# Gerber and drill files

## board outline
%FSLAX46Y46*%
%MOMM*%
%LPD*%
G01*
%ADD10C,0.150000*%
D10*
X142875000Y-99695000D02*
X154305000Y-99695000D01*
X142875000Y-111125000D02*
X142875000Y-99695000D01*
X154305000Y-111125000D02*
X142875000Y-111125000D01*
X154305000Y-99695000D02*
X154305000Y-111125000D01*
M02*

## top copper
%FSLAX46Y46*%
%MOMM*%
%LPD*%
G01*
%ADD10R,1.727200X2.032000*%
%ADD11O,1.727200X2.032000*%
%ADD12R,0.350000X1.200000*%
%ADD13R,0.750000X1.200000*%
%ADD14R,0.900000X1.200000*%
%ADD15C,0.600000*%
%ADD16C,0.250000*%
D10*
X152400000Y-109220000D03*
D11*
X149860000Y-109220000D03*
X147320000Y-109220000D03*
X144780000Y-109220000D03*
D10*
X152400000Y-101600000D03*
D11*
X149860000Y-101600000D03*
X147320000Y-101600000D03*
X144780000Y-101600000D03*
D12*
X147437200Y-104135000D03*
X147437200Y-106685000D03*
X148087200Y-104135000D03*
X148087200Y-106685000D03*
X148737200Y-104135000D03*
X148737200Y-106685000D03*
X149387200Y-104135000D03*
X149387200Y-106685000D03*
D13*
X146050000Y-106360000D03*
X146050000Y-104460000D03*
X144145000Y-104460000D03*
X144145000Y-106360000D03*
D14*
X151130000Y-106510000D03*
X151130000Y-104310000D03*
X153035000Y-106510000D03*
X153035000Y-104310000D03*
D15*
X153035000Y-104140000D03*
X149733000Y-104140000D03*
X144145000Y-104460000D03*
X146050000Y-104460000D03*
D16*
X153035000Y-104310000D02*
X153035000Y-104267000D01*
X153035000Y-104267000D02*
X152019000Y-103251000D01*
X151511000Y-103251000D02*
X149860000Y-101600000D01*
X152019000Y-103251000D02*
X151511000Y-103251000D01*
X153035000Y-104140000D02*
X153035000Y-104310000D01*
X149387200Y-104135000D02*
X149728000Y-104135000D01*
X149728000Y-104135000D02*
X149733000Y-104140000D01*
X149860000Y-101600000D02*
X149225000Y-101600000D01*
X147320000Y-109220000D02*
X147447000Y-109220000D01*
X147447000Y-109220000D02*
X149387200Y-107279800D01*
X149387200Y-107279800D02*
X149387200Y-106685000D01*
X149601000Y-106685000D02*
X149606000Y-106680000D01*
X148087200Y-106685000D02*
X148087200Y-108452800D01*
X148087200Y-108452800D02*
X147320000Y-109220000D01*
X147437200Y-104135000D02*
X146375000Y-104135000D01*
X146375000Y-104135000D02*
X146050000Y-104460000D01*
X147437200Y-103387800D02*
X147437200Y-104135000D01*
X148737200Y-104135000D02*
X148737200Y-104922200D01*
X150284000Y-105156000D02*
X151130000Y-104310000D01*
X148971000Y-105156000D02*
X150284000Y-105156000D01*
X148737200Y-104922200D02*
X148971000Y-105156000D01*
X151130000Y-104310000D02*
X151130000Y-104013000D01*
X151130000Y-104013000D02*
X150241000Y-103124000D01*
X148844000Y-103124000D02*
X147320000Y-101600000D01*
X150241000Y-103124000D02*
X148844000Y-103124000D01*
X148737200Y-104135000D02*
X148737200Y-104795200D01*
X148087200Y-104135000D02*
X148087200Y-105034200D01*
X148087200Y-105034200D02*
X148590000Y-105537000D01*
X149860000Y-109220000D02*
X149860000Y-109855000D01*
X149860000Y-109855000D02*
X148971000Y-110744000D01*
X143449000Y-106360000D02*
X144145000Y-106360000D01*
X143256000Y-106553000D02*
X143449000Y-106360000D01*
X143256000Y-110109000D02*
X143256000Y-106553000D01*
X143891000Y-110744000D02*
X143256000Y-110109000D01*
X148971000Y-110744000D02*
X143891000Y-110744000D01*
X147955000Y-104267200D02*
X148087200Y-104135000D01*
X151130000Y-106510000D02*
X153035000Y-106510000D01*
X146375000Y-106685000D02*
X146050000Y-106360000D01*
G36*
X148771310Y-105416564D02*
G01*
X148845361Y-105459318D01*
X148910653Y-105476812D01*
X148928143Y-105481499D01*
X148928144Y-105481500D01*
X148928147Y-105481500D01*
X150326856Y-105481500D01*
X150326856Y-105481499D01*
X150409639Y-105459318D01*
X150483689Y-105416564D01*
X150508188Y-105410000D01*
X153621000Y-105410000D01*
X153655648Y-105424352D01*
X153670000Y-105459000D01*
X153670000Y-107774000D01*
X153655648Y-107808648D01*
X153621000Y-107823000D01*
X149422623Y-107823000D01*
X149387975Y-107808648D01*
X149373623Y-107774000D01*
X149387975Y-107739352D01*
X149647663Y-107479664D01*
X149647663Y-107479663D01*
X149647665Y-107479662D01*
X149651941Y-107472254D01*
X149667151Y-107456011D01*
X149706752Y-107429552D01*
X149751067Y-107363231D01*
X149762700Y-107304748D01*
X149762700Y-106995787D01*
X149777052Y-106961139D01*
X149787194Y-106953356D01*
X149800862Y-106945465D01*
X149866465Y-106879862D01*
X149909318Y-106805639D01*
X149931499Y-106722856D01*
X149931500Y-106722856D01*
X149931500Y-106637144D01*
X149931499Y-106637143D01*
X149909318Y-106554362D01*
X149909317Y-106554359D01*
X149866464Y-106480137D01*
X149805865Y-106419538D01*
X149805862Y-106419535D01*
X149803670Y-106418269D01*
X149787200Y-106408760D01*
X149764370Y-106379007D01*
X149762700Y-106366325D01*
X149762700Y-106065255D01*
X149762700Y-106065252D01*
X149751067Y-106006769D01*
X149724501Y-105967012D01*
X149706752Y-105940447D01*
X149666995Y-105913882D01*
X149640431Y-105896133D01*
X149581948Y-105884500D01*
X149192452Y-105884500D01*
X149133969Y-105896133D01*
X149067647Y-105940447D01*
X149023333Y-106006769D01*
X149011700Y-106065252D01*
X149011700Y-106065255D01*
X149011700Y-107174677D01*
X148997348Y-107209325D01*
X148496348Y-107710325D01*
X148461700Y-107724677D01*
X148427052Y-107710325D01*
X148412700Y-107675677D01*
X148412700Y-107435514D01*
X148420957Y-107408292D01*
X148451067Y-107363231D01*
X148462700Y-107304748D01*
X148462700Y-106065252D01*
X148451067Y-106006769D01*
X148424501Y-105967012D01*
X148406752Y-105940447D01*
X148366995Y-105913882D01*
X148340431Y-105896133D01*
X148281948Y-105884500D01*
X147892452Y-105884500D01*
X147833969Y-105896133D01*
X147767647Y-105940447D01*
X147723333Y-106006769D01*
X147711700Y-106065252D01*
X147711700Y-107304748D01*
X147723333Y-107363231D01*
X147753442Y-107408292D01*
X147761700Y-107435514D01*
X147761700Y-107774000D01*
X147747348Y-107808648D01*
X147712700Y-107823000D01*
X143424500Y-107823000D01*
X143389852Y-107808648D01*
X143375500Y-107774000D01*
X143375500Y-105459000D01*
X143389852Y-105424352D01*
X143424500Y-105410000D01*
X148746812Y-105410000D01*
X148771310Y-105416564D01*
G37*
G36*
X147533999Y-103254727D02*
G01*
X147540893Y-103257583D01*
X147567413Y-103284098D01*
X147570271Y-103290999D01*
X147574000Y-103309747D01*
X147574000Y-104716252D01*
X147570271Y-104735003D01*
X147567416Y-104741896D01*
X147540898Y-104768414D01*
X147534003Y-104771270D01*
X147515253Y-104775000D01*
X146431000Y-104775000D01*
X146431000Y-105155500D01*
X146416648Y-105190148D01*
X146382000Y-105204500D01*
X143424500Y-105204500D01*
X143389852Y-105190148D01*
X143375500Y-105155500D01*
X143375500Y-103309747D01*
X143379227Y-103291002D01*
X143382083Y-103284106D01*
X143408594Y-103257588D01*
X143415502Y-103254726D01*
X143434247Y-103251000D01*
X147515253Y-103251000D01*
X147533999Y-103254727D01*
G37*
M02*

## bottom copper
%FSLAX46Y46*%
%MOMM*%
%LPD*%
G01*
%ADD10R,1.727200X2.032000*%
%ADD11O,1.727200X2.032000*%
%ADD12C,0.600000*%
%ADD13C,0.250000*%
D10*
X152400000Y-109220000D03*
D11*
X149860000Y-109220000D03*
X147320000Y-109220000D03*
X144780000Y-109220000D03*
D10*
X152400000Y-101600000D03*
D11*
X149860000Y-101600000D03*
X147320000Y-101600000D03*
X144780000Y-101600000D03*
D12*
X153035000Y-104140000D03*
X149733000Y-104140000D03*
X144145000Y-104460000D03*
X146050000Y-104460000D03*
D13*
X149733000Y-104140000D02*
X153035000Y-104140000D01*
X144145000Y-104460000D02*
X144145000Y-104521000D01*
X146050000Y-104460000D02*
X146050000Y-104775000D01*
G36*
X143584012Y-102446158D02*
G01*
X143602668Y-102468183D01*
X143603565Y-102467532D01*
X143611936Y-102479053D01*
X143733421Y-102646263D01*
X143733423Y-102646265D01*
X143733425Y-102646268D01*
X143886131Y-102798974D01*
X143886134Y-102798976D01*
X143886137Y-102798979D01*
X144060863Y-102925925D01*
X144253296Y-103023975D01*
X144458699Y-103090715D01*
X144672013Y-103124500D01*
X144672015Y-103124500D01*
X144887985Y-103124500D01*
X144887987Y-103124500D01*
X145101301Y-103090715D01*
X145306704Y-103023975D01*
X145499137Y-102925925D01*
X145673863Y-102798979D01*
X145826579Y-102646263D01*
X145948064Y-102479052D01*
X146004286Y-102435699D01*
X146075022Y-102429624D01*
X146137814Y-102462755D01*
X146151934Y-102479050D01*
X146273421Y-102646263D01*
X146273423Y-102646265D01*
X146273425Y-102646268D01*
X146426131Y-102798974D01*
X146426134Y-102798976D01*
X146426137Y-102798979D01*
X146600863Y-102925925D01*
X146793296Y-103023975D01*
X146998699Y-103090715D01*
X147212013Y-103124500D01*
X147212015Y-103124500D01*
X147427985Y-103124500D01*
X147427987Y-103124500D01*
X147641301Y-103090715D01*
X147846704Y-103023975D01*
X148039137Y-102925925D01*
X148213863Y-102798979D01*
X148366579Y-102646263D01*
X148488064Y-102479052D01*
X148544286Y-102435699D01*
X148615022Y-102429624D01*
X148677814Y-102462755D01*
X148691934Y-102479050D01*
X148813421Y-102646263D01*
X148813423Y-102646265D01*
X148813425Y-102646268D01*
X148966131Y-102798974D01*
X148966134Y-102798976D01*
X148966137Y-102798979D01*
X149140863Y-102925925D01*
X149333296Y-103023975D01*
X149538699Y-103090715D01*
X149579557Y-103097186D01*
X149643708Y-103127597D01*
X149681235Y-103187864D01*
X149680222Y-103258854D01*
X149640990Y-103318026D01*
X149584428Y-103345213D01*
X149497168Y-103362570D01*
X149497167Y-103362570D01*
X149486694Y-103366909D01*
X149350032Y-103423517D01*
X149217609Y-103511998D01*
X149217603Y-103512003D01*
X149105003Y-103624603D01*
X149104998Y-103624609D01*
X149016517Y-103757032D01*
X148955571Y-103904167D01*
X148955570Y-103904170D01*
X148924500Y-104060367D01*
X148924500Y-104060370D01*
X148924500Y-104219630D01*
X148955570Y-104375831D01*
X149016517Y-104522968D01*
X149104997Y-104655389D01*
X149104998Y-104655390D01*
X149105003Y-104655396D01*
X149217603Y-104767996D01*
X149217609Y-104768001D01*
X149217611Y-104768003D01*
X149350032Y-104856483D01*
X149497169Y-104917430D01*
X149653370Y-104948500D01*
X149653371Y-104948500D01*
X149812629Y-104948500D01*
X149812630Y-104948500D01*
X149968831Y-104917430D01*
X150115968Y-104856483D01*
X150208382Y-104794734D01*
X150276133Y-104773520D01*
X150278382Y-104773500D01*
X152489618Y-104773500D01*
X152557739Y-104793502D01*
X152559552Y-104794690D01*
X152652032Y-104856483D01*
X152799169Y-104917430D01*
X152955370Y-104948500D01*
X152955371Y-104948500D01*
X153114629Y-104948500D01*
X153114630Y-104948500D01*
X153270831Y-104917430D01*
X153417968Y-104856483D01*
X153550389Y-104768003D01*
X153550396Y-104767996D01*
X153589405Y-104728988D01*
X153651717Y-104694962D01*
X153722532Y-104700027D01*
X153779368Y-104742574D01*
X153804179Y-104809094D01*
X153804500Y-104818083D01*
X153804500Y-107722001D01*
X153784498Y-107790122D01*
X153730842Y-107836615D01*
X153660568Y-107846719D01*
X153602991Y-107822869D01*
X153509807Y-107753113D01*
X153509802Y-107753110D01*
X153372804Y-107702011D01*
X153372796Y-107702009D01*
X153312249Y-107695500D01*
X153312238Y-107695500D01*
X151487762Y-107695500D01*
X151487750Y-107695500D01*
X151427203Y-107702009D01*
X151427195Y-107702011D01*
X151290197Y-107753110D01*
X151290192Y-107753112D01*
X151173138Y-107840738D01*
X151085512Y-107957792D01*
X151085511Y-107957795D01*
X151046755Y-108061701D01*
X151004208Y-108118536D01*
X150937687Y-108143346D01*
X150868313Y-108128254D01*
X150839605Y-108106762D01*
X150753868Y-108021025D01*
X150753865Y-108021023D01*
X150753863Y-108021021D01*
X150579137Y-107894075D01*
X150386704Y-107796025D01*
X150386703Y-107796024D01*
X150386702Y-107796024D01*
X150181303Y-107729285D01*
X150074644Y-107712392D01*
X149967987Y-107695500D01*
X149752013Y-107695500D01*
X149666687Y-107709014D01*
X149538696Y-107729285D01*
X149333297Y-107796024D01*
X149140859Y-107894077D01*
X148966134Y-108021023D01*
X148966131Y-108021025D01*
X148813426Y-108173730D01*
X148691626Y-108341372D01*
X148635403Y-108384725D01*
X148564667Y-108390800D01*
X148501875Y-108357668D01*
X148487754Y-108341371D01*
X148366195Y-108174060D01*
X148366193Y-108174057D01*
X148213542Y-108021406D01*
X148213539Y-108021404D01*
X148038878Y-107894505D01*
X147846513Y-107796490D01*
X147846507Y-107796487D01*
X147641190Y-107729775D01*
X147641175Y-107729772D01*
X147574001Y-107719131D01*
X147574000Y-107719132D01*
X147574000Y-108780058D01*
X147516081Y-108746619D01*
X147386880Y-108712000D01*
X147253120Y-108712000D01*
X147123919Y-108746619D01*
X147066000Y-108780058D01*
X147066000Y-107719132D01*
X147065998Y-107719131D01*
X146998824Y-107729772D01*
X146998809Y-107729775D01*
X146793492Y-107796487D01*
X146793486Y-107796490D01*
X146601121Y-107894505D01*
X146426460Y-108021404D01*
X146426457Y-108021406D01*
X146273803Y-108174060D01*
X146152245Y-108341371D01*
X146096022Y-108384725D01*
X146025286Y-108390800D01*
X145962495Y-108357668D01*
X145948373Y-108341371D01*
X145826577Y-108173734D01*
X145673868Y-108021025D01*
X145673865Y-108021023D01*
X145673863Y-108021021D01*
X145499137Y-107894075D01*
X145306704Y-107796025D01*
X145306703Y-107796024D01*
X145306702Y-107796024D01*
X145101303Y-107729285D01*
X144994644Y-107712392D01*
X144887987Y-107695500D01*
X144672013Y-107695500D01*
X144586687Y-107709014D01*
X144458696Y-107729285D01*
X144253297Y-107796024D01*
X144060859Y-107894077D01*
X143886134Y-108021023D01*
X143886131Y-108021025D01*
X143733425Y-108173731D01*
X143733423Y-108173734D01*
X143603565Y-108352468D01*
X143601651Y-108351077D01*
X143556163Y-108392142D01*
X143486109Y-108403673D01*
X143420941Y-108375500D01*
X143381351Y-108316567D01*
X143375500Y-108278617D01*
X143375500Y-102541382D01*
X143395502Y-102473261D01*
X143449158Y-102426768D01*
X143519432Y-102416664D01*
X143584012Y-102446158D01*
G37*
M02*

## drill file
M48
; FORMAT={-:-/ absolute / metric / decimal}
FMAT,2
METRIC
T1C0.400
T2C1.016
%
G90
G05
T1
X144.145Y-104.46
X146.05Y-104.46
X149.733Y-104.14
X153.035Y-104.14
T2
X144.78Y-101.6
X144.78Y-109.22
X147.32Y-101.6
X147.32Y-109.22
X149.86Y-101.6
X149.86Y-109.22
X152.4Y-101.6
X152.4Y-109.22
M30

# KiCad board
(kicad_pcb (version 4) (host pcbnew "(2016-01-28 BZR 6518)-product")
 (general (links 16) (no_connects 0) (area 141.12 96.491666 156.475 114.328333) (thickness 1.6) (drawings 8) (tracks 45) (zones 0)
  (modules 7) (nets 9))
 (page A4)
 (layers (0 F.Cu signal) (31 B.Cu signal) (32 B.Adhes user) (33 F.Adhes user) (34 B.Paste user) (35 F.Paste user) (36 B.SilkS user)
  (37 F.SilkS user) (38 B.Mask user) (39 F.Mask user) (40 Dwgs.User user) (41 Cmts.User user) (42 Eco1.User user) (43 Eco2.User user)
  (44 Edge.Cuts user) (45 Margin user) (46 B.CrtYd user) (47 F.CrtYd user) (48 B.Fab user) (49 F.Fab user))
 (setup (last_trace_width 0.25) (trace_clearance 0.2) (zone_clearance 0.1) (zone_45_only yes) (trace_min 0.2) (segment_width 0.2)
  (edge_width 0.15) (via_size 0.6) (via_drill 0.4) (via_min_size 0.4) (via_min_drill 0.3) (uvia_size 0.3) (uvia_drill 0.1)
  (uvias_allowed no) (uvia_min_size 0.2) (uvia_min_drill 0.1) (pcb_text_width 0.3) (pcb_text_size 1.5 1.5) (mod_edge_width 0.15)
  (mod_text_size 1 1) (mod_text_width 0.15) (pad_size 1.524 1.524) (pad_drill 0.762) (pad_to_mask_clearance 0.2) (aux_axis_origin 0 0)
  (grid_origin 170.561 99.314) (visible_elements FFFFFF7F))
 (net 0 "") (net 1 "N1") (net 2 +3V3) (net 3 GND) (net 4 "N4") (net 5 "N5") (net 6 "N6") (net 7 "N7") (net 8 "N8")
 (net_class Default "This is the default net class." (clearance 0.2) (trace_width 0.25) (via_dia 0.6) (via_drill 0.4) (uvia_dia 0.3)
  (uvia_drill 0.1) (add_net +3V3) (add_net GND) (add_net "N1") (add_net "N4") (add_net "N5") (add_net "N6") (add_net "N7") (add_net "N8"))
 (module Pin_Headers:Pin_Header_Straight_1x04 (layer F.Cu) (at 152.4 109.22 270)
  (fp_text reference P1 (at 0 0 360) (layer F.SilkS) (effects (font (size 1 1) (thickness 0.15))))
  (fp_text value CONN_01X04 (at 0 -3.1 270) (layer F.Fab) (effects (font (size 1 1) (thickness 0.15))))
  (pad 1 thru_hole rect (at 0 0 270) (size 2.032 1.7272) (drill 1.016) (layers *.Cu *.Mask F.SilkS) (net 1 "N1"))
  (pad 2 thru_hole oval (at 0 2.54 270) (size 2.032 1.7272) (drill 1.016) (layers *.Cu *.Mask F.SilkS) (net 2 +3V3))
  (pad 3 thru_hole oval (at 0 5.08 270) (size 2.032 1.7272) (drill 1.016) (layers *.Cu *.Mask F.SilkS) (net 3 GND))
  (pad 4 thru_hole oval (at 0 7.62 270) (size 2.032 1.7272) (drill 1.016) (layers *.Cu *.Mask F.SilkS) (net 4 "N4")))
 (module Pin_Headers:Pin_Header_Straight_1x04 (layer F.Cu) (at 152.4 101.6 270)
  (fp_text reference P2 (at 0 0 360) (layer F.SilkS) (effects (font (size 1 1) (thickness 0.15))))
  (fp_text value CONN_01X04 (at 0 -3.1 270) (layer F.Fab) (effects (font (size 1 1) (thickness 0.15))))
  (pad 1 thru_hole rect (at 0 0 270) (size 2.032 1.7272) (drill 1.016) (layers *.Cu *.Mask F.SilkS) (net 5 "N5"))
  (pad 2 thru_hole oval (at 0 2.54 270) (size 2.032 1.7272) (drill 1.016) (layers *.Cu *.Mask F.SilkS) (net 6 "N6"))
  (pad 3 thru_hole oval (at 0 5.08 270) (size 2.032 1.7272) (drill 1.016) (layers *.Cu *.Mask F.SilkS) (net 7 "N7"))
  (pad 4 thru_hole oval (at 0 7.62 270) (size 2.032 1.7272) (drill 1.016) (layers *.Cu *.Mask F.SilkS) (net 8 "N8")))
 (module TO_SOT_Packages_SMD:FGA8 (layer F.Cu) (at 148.4122 105.41) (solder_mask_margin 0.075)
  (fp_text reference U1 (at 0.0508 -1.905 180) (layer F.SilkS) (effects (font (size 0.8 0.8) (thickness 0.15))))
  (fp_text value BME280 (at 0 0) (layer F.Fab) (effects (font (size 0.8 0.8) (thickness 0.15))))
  (pad 1 smd rect (at -0.975 -1.275) (size 0.35 1.2) (layers F.Cu F.Paste F.Mask) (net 3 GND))
  (pad 8 smd rect (at -0.975 1.275) (size 0.35 1.2) (layers F.Cu F.Paste F.Mask) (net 2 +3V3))
  (pad 2 smd rect (at -0.325 -1.275) (size 0.35 1.2) (layers F.Cu F.Paste F.Mask) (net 2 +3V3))
  (pad 7 smd rect (at -0.325 1.275) (size 0.35 1.2) (layers F.Cu F.Paste F.Mask) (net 3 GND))
  (pad 3 smd rect (at 0.325 -1.275) (size 0.35 1.2) (layers F.Cu F.Paste F.Mask) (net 7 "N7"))
  (pad 6 smd rect (at 0.325 1.275) (size 0.35 1.2) (layers F.Cu F.Paste F.Mask) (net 2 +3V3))
  (pad 4 smd rect (at 0.975 -1.275) (size 0.35 1.2) (layers F.Cu F.Paste F.Mask) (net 6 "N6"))
  (pad 5 smd rect (at 0.975 1.275) (size 0.35 1.2) (layers F.Cu F.Paste F.Mask) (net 3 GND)))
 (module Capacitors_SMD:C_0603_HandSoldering (layer F.Cu) (at 146.05 105.41 90)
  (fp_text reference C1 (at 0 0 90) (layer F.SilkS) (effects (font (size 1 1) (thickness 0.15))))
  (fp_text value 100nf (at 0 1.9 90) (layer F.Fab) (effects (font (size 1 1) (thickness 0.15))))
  (pad 1 smd rect (at -0.95 0 90) (size 1.2 0.75) (layers F.Cu F.Paste F.Mask) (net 2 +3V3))
  (pad 2 smd rect (at 0.95 0 90) (size 1.2 0.75) (layers F.Cu F.Paste F.Mask) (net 3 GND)))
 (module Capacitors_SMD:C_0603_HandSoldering (layer F.Cu) (at 144.145 105.41 270)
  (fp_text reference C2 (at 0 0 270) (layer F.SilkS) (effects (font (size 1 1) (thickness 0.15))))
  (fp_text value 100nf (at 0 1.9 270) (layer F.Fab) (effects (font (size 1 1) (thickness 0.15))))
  (pad 1 smd rect (at -0.95 0 270) (size 1.2 0.75) (layers F.Cu F.Paste F.Mask) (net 3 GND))
  (pad 2 smd rect (at 0.95 0 270) (size 1.2 0.75) (layers F.Cu F.Paste F.Mask) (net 2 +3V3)))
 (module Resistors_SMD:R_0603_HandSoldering (layer F.Cu) (at 151.13 105.41 90)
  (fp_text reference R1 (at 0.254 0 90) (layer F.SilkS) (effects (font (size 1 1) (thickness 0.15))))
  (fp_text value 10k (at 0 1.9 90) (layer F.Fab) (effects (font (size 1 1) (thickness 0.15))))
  (pad 1 smd rect (at -1.1 0 90) (size 1.2 0.9) (layers F.Cu F.Paste F.Mask) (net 2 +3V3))
  (pad 2 smd rect (at 1.1 0 90) (size 1.2 0.9) (layers F.Cu F.Paste F.Mask) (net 7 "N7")))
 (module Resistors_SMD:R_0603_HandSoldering (layer F.Cu) (at 153.035 105.41 90)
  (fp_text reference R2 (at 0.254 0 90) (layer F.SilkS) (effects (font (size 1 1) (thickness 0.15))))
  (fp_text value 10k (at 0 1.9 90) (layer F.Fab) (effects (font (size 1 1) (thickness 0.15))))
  (pad 1 smd rect (at -1.1 0 90) (size 1.2 0.9) (layers F.Cu F.Paste F.Mask) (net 2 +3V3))
  (pad 2 smd rect (at 1.1 0 90) (size 1.2 0.9) (layers F.Cu F.Paste F.Mask) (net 6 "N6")))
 (gr_line (start 142.875 99.695) (end 154.305 99.695) (angle 90) (layer Edge.Cuts) (width 0.15))
 (gr_line (start 142.875 111.125) (end 142.875 99.695) (angle 90) (layer Edge.Cuts) (width 0.15))
 (gr_line (start 154.305 111.125) (end 142.875 111.125) (angle 90) (layer Edge.Cuts) (width 0.15))
 (gr_line (start 154.305 99.695) (end 154.305 111.125) (angle 90) (layer Edge.Cuts) (width 0.15))
 (segment (start 153.035 104.31) (end 153.035 104.267) (width 0.25) (layer F.Cu) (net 6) (status C00000))
 (segment (start 153.035 104.267) (end 152.019 103.251) (width 0.25) (layer F.Cu) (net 6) (status 400000))
 (segment (start 151.511 103.251) (end 149.86 101.6) (width 0.25) (layer F.Cu) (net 6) (status 800000))
 (segment (start 152.019 103.251) (end 151.511 103.251) (width 0.25) (layer F.Cu) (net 6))
 (via (at 153.035 104.14) (size 0.6) (drill 0.4) (layers F.Cu B.Cu) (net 6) (status 800000))
 (segment (start 153.035 104.14) (end 153.035 104.31) (width 0.25) (layer F.Cu) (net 6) (status C00000))
 (segment (start 149.3872 104.135) (end 149.728 104.135) (width 0.25) (layer F.Cu) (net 6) (status 400000))
 (segment (start 149.733 104.14) (end 153.035 104.14) (width 0.25) (layer B.Cu) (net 6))
 (via (at 149.733 104.14) (size 0.6) (drill 0.4) (layers F.Cu B.Cu) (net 6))
 (segment (start 149.728 104.135) (end 149.733 104.14) (width 0.25) (layer F.Cu) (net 6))
 (segment (start 149.86 101.6) (end 149.225 101.6) (width 0.25) (layer F.Cu) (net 6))
 (via (at 144.145 104.46) (size 0.6) (drill 0.4) (layers F.Cu B.Cu) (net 3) (status C00000))
 (segment (start 144.145 104.46) (end 144.145 104.521) (width 0.25) (layer B.Cu) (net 3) (status 400000))
 (segment (start 147.32 109.22) (end 147.447 109.22) (width 0.25) (layer F.Cu) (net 3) (status C00000))
 (segment (start 147.447 109.22) (end 149.3872 107.2798) (width 0.25) (layer F.Cu) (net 3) (status C00000))
 (segment (start 149.3872 107.2798) (end 149.3872 106.685) (width 0.25) (layer F.Cu) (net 3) (status C00000))
 (segment (start 149.601 106.685) (end 149.606 106.68) (width 0.25) (layer F.Cu) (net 3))
 (segment (start 148.0872 106.685) (end 148.0872 108.4528) (width 0.25) (layer F.Cu) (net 3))
 (segment (start 148.0872 108.4528) (end 147.32 109.22) (width 0.25) (layer F.Cu) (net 3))
 (segment (start 147.4372 104.135) (end 146.375 104.135) (width 0.25) (layer F.Cu) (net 3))
 (segment (start 146.375 104.135) (end 146.05 104.46) (width 0.25) (layer F.Cu) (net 3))
 (via (at 146.05 104.46) (size 0.6) (drill 0.4) (layers F.Cu B.Cu) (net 3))
 (segment (start 146.05 104.46) (end 146.05 104.775) (width 0.25) (layer B.Cu) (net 3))
 (segment (start 147.4372 103.3878) (end 147.4372 104.135) (width 0.25) (layer F.Cu) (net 3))
 (segment (start 148.7372 104.135) (end 148.7372 104.9222) (width 0.25) (layer F.Cu) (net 7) (status 400000))
 (segment (start 150.284 105.156) (end 151.13 104.31) (width 0.25) (layer F.Cu) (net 7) (status 800000))
 (segment (start 148.971 105.156) (end 150.284 105.156) (width 0.25) (layer F.Cu) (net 7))
 (segment (start 148.7372 104.9222) (end 148.971 105.156) (width 0.25) (layer F.Cu) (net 7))
 (segment (start 151.13 104.31) (end 151.13 104.013) (width 0.25) (layer F.Cu) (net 7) (status C00000))
 (segment (start 151.13 104.013) (end 150.241 103.124) (width 0.25) (layer F.Cu) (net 7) (status 400000))
 (segment (start 148.844 103.124) (end 147.32 101.6) (width 0.25) (layer F.Cu) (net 7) (status 800000))
 (segment (start 150.241 103.124) (end 148.844 103.124) (width 0.25) (layer F.Cu) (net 7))
 (segment (start 148.7372 104.135) (end 148.7372 104.7952) (width 0.25) (layer F.Cu) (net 7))
 (segment (start 148.0872 104.135) (end 148.0872 105.0342) (width 0.25) (layer F.Cu) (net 2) (status 400000))
 (segment (start 148.0872 105.0342) (end 148.59 105.537) (width 0.25) (layer F.Cu) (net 2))
 (segment (start 149.86 109.22) (end 149.86 109.855) (width 0.25) (layer F.Cu) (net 2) (status C00000))
 (segment (start 149.86 109.855) (end 148.971 110.744) (width 0.25) (layer F.Cu) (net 2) (status 400000))
 (segment (start 143.449 106.36) (end 144.145 106.36) (width 0.25) (layer F.Cu) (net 2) (status 800000))
 (segment (start 143.256 106.553) (end 143.449 106.36) (width 0.25) (layer F.Cu) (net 2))
 (segment (start 143.256 110.109) (end 143.256 106.553) (width 0.25) (layer F.Cu) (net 2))
 (segment (start 143.891 110.744) (end 143.256 110.109) (width 0.25) (layer F.Cu) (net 2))
 (segment (start 148.971 110.744) (end 143.891 110.744) (width 0.25) (layer F.Cu) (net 2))
 (segment (start 147.955 104.2672) (end 148.0872 104.135) (width 0.25) (layer F.Cu) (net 2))
 (segment (start 151.13 106.51) (end 153.035 106.51) (width 0.25) (layer F.Cu) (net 2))
 (segment (start 146.375 106.685) (end 146.05 106.36) (width 0.25) (layer F.Cu) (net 2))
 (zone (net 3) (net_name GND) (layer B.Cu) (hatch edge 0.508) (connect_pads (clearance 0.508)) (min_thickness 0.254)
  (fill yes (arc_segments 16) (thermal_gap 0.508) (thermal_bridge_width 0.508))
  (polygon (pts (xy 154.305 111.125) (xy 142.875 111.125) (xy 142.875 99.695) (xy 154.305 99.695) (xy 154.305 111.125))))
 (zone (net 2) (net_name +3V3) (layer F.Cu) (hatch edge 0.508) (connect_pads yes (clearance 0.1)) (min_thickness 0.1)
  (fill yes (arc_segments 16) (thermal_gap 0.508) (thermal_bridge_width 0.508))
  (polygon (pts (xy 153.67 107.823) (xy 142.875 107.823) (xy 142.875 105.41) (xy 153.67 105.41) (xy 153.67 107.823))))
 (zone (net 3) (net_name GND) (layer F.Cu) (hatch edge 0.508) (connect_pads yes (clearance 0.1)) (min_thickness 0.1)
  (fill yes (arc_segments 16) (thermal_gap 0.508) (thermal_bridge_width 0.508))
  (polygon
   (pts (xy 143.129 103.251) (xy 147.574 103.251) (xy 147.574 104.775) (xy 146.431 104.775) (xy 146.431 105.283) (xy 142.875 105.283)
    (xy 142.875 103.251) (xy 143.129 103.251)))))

